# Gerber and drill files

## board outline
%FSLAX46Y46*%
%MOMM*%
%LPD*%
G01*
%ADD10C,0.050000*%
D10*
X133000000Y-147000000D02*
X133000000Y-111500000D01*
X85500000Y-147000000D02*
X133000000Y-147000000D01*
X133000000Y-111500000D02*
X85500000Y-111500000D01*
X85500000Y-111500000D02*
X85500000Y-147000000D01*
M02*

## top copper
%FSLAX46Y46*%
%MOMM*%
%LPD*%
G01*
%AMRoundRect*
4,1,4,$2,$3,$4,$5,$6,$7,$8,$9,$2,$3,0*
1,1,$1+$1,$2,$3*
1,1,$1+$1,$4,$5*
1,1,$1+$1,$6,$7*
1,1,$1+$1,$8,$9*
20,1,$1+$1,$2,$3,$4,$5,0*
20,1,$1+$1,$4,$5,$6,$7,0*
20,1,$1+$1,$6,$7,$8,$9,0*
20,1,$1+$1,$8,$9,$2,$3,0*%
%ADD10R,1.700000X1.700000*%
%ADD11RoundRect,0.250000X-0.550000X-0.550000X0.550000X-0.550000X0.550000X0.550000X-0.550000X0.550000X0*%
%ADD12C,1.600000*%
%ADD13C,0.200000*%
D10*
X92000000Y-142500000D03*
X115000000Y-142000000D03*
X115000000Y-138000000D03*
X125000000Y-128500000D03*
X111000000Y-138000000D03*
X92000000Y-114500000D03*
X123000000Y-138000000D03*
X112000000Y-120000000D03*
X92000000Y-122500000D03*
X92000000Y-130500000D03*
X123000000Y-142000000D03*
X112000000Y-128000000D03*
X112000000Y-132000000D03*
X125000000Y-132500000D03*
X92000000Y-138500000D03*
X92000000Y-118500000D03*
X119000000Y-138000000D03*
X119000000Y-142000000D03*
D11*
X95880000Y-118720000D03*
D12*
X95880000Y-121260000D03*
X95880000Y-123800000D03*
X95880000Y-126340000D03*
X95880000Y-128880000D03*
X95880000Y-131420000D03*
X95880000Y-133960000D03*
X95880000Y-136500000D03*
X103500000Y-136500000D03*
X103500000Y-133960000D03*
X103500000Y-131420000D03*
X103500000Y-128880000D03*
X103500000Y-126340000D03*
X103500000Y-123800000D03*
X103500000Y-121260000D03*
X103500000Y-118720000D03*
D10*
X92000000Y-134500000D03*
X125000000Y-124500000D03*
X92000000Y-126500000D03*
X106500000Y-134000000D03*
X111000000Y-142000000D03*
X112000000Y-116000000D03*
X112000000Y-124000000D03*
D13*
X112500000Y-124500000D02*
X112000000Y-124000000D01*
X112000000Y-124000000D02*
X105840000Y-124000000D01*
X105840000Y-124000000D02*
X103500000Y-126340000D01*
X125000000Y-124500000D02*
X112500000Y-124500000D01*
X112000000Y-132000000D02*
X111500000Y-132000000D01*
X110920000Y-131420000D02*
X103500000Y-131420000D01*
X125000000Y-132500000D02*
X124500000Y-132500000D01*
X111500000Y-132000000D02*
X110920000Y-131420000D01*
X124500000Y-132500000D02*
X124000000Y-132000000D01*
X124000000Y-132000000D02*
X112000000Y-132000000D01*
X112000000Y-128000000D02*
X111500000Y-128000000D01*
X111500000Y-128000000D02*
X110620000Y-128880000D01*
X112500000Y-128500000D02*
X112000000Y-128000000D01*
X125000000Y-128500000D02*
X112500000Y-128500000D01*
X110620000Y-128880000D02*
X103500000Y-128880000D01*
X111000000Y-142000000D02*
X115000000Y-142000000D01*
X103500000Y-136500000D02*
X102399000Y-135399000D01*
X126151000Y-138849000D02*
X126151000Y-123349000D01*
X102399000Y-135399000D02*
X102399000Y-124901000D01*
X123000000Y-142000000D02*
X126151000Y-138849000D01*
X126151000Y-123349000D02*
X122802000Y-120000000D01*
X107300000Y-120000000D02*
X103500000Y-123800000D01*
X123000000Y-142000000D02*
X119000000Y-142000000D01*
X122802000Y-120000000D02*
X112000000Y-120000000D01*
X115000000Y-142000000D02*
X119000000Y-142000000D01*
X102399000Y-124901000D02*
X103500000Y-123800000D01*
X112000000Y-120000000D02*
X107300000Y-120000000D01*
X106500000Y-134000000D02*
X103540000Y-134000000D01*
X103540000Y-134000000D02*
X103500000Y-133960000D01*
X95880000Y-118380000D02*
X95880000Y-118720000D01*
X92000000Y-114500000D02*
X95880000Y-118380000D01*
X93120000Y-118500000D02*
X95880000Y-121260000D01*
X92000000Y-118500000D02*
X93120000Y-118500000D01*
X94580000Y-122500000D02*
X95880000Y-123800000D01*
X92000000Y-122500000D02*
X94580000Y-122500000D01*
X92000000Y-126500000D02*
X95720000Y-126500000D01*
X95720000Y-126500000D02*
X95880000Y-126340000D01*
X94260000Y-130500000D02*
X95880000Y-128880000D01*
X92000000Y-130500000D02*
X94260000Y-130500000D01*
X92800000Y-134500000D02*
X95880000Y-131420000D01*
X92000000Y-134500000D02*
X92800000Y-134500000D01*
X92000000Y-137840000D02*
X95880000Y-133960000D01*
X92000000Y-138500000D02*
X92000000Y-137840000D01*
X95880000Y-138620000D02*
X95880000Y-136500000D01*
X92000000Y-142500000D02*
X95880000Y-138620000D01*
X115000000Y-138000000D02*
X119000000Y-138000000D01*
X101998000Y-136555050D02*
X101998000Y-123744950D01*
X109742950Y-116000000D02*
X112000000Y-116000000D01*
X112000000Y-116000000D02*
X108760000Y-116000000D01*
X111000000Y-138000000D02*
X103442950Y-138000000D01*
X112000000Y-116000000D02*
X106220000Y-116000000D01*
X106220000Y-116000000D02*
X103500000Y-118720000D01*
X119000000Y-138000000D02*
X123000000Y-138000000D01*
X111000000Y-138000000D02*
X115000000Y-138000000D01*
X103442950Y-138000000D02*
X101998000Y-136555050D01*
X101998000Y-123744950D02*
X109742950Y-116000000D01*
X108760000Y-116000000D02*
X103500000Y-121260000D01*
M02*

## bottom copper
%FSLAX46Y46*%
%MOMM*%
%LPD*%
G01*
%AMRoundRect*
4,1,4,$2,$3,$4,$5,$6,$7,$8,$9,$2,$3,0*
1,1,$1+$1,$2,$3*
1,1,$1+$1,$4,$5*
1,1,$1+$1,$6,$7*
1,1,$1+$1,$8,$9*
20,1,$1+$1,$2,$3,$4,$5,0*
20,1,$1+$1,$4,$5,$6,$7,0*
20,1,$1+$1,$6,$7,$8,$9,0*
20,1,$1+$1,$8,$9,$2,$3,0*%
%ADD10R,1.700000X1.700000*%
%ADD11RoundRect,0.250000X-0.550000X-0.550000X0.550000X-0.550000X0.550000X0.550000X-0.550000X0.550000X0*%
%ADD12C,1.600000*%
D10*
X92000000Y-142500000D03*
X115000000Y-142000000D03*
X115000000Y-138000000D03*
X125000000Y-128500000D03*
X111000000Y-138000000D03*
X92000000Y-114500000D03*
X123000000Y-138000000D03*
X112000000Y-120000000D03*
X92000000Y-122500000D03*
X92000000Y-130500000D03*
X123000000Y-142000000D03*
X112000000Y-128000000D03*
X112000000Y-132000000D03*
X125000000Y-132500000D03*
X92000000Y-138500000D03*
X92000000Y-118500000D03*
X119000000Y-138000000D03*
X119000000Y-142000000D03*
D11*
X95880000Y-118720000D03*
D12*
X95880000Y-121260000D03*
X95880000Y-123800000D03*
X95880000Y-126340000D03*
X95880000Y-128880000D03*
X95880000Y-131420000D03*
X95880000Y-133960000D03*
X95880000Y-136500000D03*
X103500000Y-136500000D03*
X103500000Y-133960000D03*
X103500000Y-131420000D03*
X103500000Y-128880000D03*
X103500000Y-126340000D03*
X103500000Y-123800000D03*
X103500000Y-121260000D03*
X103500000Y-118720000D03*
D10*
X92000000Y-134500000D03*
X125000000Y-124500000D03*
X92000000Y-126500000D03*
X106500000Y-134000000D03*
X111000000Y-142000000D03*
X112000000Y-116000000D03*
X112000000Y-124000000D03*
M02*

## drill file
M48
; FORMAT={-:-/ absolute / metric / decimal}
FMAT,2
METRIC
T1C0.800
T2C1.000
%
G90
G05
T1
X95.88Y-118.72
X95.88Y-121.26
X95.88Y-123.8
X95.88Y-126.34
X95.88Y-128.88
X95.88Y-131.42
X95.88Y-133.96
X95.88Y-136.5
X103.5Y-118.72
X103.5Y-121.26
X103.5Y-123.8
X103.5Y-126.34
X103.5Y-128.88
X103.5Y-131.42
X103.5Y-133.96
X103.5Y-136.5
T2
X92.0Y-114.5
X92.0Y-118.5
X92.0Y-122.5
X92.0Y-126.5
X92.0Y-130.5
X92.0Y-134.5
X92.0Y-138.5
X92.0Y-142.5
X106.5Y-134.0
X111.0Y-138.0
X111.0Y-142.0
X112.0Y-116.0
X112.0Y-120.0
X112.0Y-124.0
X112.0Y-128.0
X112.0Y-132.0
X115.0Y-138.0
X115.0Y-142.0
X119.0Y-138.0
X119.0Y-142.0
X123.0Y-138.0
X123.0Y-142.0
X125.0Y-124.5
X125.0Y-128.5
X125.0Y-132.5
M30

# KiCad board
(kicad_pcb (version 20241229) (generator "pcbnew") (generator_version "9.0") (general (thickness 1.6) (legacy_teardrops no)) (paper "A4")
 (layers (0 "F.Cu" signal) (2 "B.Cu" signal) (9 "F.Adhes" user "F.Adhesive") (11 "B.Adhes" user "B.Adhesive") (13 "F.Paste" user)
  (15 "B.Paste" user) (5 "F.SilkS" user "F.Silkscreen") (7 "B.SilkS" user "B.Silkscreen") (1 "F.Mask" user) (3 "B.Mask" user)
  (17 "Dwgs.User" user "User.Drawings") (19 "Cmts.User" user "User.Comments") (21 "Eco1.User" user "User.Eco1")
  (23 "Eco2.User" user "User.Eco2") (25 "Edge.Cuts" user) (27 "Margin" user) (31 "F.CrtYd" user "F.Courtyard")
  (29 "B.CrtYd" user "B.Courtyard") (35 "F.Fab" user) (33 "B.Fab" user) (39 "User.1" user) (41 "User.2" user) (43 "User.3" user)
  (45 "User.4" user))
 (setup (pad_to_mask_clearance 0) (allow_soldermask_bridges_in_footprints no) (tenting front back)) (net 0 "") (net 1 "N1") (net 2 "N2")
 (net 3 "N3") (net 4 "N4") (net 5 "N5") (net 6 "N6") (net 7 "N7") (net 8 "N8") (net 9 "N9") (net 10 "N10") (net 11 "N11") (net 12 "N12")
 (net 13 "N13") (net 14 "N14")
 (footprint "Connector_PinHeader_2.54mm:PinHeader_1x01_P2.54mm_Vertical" (layer "F.Cu") (at 92 142.5)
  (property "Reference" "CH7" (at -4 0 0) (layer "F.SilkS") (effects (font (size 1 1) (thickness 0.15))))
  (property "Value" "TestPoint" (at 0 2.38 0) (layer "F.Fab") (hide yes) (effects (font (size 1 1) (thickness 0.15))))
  (pad "1" thru_hole rect (at 0 0) (size 1.7 1.7) (drill 1) (layers "*.Cu" "*.Mask") (remove_unused_layers no) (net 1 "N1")))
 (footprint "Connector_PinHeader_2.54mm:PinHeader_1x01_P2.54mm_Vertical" (layer "F.Cu") (at 115 142)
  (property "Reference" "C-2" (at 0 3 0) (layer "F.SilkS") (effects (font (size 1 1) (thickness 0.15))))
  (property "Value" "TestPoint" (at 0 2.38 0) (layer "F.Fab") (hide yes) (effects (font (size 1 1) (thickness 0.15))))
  (pad "1" thru_hole rect (at 0 0) (size 1.7 1.7) (drill 1) (layers "*.Cu" "*.Mask") (remove_unused_layers no) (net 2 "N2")))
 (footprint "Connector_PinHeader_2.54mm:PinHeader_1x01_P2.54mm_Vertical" (layer "F.Cu") (at 115 138)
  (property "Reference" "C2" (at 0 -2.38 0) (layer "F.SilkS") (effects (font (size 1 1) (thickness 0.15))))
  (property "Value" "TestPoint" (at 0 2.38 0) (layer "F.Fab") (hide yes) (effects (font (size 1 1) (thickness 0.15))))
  (pad "1" thru_hole rect (at 0 0) (size 1.7 1.7) (drill 1) (layers "*.Cu" "*.Mask") (remove_unused_layers no) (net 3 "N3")))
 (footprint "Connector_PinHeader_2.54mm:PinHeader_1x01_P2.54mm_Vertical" (layer "F.Cu") (at 125 128.5)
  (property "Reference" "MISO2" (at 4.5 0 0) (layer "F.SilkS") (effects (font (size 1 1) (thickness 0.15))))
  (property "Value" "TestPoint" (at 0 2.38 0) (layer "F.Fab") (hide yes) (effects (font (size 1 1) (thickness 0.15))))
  (pad "1" thru_hole rect (at 0 0) (size 1.7 1.7) (drill 1) (layers "*.Cu" "*.Mask") (remove_unused_layers no) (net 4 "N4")))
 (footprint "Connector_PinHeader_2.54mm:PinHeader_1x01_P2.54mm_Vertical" (layer "F.Cu") (at 111 138)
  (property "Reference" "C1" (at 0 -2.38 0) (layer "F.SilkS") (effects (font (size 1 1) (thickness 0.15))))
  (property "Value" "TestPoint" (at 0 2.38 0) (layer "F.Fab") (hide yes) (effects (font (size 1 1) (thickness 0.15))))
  (pad "1" thru_hole rect (at 0 0) (size 1.7 1.7) (drill 1) (layers "*.Cu" "*.Mask") (remove_unused_layers no) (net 3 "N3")))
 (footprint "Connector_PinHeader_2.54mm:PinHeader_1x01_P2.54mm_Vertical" (layer "F.Cu") (at 92 114.5)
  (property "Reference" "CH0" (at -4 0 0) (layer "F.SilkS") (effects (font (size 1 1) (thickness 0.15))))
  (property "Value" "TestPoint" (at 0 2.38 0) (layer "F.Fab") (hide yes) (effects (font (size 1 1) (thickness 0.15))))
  (pad "1" thru_hole rect (at 0 0) (size 1.7 1.7) (drill 1) (layers "*.Cu" "*.Mask") (remove_unused_layers no) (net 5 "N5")))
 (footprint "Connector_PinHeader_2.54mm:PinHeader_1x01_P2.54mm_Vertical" (layer "F.Cu") (at 123 138)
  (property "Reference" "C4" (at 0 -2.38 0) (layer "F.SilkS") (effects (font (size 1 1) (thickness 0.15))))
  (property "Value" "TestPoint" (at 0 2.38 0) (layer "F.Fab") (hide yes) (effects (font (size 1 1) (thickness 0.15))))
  (pad "1" thru_hole rect (at 0 0) (size 1.7 1.7) (drill 1) (layers "*.Cu" "*.Mask") (remove_unused_layers no) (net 3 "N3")))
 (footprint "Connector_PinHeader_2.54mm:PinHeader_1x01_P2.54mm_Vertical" (layer "F.Cu") (at 112 120)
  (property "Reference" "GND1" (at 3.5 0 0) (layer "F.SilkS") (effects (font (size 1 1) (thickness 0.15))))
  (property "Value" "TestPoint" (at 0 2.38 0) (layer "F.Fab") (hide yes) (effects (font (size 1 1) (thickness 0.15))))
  (pad "1" thru_hole rect (at 0 0) (size 1.7 1.7) (drill 1) (layers "*.Cu" "*.Mask") (remove_unused_layers no) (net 2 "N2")))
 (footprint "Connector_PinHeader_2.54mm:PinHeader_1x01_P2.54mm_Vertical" (layer "F.Cu") (at 92 122.5)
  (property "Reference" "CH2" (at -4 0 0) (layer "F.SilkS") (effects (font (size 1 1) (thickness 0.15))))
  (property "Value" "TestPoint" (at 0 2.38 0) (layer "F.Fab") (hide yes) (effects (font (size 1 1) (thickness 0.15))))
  (pad "1" thru_hole rect (at 0 0) (size 1.7 1.7) (drill 1) (layers "*.Cu" "*.Mask") (remove_unused_layers no) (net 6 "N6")))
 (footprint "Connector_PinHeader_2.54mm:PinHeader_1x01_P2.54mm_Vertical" (layer "F.Cu") (at 92 130.5)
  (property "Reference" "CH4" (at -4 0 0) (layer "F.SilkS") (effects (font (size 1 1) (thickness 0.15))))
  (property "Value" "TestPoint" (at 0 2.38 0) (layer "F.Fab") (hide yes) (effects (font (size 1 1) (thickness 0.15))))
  (pad "1" thru_hole rect (at 0 0) (size 1.7 1.7) (drill 1) (layers "*.Cu" "*.Mask") (remove_unused_layers no) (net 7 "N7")))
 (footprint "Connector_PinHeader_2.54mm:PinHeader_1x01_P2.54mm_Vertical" (layer "F.Cu") (at 123 142)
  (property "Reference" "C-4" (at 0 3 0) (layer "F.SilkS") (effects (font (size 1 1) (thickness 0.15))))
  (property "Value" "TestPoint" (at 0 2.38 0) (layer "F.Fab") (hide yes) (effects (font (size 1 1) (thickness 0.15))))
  (pad "1" thru_hole rect (at 0 0) (size 1.7 1.7) (drill 1) (layers "*.Cu" "*.Mask") (remove_unused_layers no) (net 2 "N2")))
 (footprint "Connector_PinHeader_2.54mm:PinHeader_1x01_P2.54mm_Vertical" (layer "F.Cu") (at 112 128)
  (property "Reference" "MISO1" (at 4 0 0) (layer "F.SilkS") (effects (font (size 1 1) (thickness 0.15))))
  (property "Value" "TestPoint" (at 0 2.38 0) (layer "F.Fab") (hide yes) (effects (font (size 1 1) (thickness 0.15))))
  (pad "1" thru_hole rect (at 0 0) (size 1.7 1.7) (drill 1) (layers "*.Cu" "*.Mask") (remove_unused_layers no) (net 4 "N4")))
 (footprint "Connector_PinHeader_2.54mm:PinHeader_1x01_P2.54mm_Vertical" (layer "F.Cu") (at 112 132)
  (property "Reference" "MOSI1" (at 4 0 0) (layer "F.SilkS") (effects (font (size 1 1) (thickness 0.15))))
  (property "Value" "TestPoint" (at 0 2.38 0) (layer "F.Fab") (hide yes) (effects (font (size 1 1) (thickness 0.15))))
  (pad "1" thru_hole rect (at 0 0) (size 1.7 1.7) (drill 1) (layers "*.Cu" "*.Mask") (remove_unused_layers no) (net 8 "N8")))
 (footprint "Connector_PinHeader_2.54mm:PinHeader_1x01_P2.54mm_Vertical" (layer "F.Cu") (at 125 132.5)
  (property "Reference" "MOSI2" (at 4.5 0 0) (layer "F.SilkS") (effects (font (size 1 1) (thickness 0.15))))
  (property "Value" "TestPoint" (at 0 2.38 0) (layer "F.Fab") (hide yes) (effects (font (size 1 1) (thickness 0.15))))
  (pad "1" thru_hole rect (at 0 0) (size 1.7 1.7) (drill 1) (layers "*.Cu" "*.Mask") (remove_unused_layers no) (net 8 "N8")))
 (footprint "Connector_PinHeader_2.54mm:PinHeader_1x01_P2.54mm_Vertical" (layer "F.Cu") (at 92 138.5)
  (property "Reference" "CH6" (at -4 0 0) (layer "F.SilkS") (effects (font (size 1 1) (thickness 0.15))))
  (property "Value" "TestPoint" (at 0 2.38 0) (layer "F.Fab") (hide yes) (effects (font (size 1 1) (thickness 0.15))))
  (pad "1" thru_hole rect (at 0 0) (size 1.7 1.7) (drill 1) (layers "*.Cu" "*.Mask") (remove_unused_layers no) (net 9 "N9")))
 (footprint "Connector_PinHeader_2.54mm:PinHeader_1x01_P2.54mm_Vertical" (layer "F.Cu") (at 92 118.5)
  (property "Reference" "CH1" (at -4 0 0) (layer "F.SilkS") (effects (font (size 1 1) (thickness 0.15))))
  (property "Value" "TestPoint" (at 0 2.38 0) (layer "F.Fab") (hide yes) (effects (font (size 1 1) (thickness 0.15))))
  (pad "1" thru_hole rect (at 0 0) (size 1.7 1.7) (drill 1) (layers "*.Cu" "*.Mask") (remove_unused_layers no) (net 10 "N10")))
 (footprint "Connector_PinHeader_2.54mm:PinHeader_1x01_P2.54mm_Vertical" (layer "F.Cu") (at 119 138)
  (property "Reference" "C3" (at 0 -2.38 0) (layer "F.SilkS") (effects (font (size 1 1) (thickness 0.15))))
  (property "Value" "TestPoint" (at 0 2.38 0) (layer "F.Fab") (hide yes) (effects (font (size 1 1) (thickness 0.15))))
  (pad "1" thru_hole rect (at 0 0) (size 1.7 1.7) (drill 1) (layers "*.Cu" "*.Mask") (remove_unused_layers no) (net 3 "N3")))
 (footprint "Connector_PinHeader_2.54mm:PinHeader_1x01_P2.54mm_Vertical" (layer "F.Cu") (at 119 142)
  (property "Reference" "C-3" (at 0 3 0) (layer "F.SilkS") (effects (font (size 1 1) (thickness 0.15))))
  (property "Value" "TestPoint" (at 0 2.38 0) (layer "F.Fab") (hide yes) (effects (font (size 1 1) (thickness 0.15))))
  (pad "1" thru_hole rect (at 0 0) (size 1.7 1.7) (drill 1) (layers "*.Cu" "*.Mask") (remove_unused_layers no) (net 2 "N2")))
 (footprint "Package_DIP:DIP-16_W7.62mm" (layer "F.Cu") (at 95.88 118.72)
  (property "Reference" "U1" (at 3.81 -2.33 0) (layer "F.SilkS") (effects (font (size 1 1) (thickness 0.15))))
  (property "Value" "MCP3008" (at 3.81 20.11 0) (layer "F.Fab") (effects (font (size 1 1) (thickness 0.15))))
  (pad "1" thru_hole roundrect (at 0 0) (size 1.6 1.6) (drill 0.8) (layers "*.Cu" "*.Mask") (remove_unused_layers no)
   (roundrect_rratio 0.15625) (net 5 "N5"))
  (pad "2" thru_hole circle (at 0 2.54) (size 1.6 1.6) (drill 0.8) (layers "*.Cu" "*.Mask") (remove_unused_layers no) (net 10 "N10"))
  (pad "3" thru_hole circle (at 0 5.08) (size 1.6 1.6) (drill 0.8) (layers "*.Cu" "*.Mask") (remove_unused_layers no) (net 6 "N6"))
  (pad "4" thru_hole circle (at 0 7.62) (size 1.6 1.6) (drill 0.8) (layers "*.Cu" "*.Mask") (remove_unused_layers no) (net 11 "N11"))
  (pad "5" thru_hole circle (at 0 10.16) (size 1.6 1.6) (drill 0.8) (layers "*.Cu" "*.Mask") (remove_unused_layers no) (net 7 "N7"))
  (pad "6" thru_hole circle (at 0 12.7) (size 1.6 1.6) (drill 0.8) (layers "*.Cu" "*.Mask") (remove_unused_layers no) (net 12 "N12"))
  (pad "7" thru_hole circle (at 0 15.24) (size 1.6 1.6) (drill 0.8) (layers "*.Cu" "*.Mask") (remove_unused_layers no) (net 9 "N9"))
  (pad "8" thru_hole circle (at 0 17.78) (size 1.6 1.6) (drill 0.8) (layers "*.Cu" "*.Mask") (remove_unused_layers no) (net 1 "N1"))
  (pad "9" thru_hole circle (at 7.62 17.78) (size 1.6 1.6) (drill 0.8) (layers "*.Cu" "*.Mask") (remove_unused_layers no) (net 2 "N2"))
  (pad "10" thru_hole circle (at 7.62 15.24) (size 1.6 1.6) (drill 0.8) (layers "*.Cu" "*.Mask") (remove_unused_layers no) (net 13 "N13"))
  (pad "11" thru_hole circle (at 7.62 12.7) (size 1.6 1.6) (drill 0.8) (layers "*.Cu" "*.Mask") (remove_unused_layers no) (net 8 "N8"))
  (pad "12" thru_hole circle (at 7.62 10.16) (size 1.6 1.6) (drill 0.8) (layers "*.Cu" "*.Mask") (remove_unused_layers no) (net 4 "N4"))
  (pad "13" thru_hole circle (at 7.62 7.62) (size 1.6 1.6) (drill 0.8) (layers "*.Cu" "*.Mask") (remove_unused_layers no) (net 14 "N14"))
  (pad "14" thru_hole circle (at 7.62 5.08) (size 1.6 1.6) (drill 0.8) (layers "*.Cu" "*.Mask") (remove_unused_layers no) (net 2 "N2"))
  (pad "15" thru_hole circle (at 7.62 2.54) (size 1.6 1.6) (drill 0.8) (layers "*.Cu" "*.Mask") (remove_unused_layers no) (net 3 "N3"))
  (pad "16" thru_hole circle (at 7.62 0) (size 1.6 1.6) (drill 0.8) (layers "*.Cu" "*.Mask") (remove_unused_layers no) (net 3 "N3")))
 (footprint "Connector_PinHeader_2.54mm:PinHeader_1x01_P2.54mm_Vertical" (layer "F.Cu") (at 92 134.5)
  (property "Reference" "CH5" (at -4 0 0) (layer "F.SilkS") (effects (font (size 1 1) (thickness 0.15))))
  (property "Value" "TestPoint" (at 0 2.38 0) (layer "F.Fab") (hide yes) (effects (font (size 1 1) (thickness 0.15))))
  (pad "1" thru_hole rect (at 0 0) (size 1.7 1.7) (drill 1) (layers "*.Cu" "*.Mask") (remove_unused_layers no) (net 12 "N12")))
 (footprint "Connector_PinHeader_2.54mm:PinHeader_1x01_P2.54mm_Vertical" (layer "F.Cu") (at 125 124.5)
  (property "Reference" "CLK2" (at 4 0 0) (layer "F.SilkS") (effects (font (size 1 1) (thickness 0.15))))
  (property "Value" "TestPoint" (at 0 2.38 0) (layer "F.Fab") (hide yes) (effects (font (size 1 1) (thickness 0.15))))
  (pad "1" thru_hole rect (at 0 0) (size 1.7 1.7) (drill 1) (layers "*.Cu" "*.Mask") (remove_unused_layers no) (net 14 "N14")))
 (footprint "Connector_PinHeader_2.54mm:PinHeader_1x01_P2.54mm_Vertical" (layer "F.Cu") (at 92 126.5)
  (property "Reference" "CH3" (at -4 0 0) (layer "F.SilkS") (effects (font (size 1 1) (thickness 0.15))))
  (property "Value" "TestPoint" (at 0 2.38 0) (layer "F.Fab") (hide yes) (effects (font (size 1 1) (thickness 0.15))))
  (pad "1" thru_hole rect (at 0 0) (size 1.7 1.7) (drill 1) (layers "*.Cu" "*.Mask") (remove_unused_layers no) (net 11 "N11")))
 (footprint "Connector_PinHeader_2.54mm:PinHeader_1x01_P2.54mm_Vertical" (layer "F.Cu") (at 106.5 134)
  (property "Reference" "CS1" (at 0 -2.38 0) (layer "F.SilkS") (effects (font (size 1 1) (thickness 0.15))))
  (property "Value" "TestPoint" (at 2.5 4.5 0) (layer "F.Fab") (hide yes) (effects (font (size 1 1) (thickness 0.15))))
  (pad "1" thru_hole rect (at 0 0) (size 1.7 1.7) (drill 1) (layers "*.Cu" "*.Mask") (remove_unused_layers no) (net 13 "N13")))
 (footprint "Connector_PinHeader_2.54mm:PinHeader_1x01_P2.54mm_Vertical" (layer "F.Cu") (at 111 142)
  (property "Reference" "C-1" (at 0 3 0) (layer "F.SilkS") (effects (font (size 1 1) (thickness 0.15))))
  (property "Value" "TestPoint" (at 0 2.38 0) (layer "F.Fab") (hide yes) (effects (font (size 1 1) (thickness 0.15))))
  (pad "1" thru_hole rect (at 0 0) (size 1.7 1.7) (drill 1) (layers "*.Cu" "*.Mask") (remove_unused_layers no) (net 2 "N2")))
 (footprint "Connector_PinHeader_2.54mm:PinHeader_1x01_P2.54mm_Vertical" (layer "F.Cu") (at 112 116)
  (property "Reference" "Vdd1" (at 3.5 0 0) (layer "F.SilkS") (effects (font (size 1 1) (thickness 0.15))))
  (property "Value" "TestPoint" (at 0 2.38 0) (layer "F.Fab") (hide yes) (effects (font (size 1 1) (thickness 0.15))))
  (pad "1" thru_hole rect (at 0 0) (size 1.7 1.7) (drill 1) (layers "*.Cu" "*.Mask") (remove_unused_layers no) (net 3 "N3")))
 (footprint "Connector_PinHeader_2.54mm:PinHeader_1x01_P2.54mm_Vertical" (layer "F.Cu") (at 112 124)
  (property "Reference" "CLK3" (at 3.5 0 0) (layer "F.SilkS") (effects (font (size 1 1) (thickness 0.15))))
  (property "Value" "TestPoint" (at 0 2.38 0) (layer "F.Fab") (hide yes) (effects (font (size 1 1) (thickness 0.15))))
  (pad "1" thru_hole rect (at 0 0) (size 1.7 1.7) (drill 1) (layers "*.Cu" "*.Mask") (remove_unused_layers no) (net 14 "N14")))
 (gr_line (start 133 147) (end 133 111.5) (stroke (width 0.05) (type default)) (layer "Edge.Cuts"))
 (gr_line (start 85.5 147) (end 133 147) (stroke (width 0.05) (type default)) (layer "Edge.Cuts"))
 (gr_line (start 133 111.5) (end 85.5 111.5) (stroke (width 0.05) (type default)) (layer "Edge.Cuts"))
 (gr_line (start 85.5 111.5) (end 85.5 147) (stroke (width 0.05) (type default)) (layer "Edge.Cuts"))
 (segment (start 112.5 124.5) (end 112 124) (width 0.2) (layer "F.Cu") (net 14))
 (segment (start 112 124) (end 105.84 124) (width 0.2) (layer "F.Cu") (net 14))
 (segment (start 105.84 124) (end 103.5 126.34) (width 0.2) (layer "F.Cu") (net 14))
 (segment (start 125 124.5) (end 112.5 124.5) (width 0.2) (layer "F.Cu") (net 14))
 (segment (start 112 132) (end 111.5 132) (width 0.2) (layer "F.Cu") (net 8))
 (segment (start 110.92 131.42) (end 103.5 131.42) (width 0.2) (layer "F.Cu") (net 8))
 (segment (start 125 132.5) (end 124.5 132.5) (width 0.2) (layer "F.Cu") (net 8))
 (segment (start 111.5 132) (end 110.92 131.42) (width 0.2) (layer "F.Cu") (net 8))
 (segment (start 124.5 132.5) (end 124 132) (width 0.2) (layer "F.Cu") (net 8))
 (segment (start 124 132) (end 112 132) (width 0.2) (layer "F.Cu") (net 8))
 (segment (start 112 128) (end 111.5 128) (width 0.2) (layer "F.Cu") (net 4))
 (segment (start 111.5 128) (end 110.62 128.88) (width 0.2) (layer "F.Cu") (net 4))
 (segment (start 112.5 128.5) (end 112 128) (width 0.2) (layer "F.Cu") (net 4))
 (segment (start 125 128.5) (end 112.5 128.5) (width 0.2) (layer "F.Cu") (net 4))
 (segment (start 110.62 128.88) (end 103.5 128.88) (width 0.2) (layer "F.Cu") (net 4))
 (segment (start 111 142) (end 115 142) (width 0.2) (layer "F.Cu") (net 2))
 (segment (start 103.5 136.5) (end 102.399 135.399) (width 0.2) (layer "F.Cu") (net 2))
 (segment (start 126.151 138.849) (end 126.151 123.349) (width 0.2) (layer "F.Cu") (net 2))
 (segment (start 102.399 135.399) (end 102.399 124.901) (width 0.2) (layer "F.Cu") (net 2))
 (segment (start 123 142) (end 126.151 138.849) (width 0.2) (layer "F.Cu") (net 2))
 (segment (start 126.151 123.349) (end 122.802 120) (width 0.2) (layer "F.Cu") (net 2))
 (segment (start 107.3 120) (end 103.5 123.8) (width 0.2) (layer "F.Cu") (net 2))
 (segment (start 123 142) (end 119 142) (width 0.2) (layer "F.Cu") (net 2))
 (segment (start 122.802 120) (end 112 120) (width 0.2) (layer "F.Cu") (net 2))
 (segment (start 115 142) (end 119 142) (width 0.2) (layer "F.Cu") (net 2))
 (segment (start 102.399 124.901) (end 103.5 123.8) (width 0.2) (layer "F.Cu") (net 2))
 (segment (start 112 120) (end 107.3 120) (width 0.2) (layer "F.Cu") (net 2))
 (segment (start 106.5 134) (end 103.54 134) (width 0.2) (layer "F.Cu") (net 13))
 (segment (start 103.54 134) (end 103.5 133.96) (width 0.2) (layer "F.Cu") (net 13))
 (segment (start 95.88 118.38) (end 95.88 118.72) (width 0.2) (layer "F.Cu") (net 5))
 (segment (start 92 114.5) (end 95.88 118.38) (width 0.2) (layer "F.Cu") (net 5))
 (segment (start 93.12 118.5) (end 95.88 121.26) (width 0.2) (layer "F.Cu") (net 10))
 (segment (start 92 118.5) (end 93.12 118.5) (width 0.2) (layer "F.Cu") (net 10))
 (segment (start 94.58 122.5) (end 95.88 123.8) (width 0.2) (layer "F.Cu") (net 6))
 (segment (start 92 122.5) (end 94.58 122.5) (width 0.2) (layer "F.Cu") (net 6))
 (segment (start 92 126.5) (end 95.72 126.5) (width 0.2) (layer "F.Cu") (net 11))
 (segment (start 95.72 126.5) (end 95.88 126.34) (width 0.2) (layer "F.Cu") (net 11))
 (segment (start 94.26 130.5) (end 95.88 128.88) (width 0.2) (layer "F.Cu") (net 7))
 (segment (start 92 130.5) (end 94.26 130.5) (width 0.2) (layer "F.Cu") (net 7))
 (segment (start 92.8 134.5) (end 95.88 131.42) (width 0.2) (layer "F.Cu") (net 12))
 (segment (start 92 134.5) (end 92.8 134.5) (width 0.2) (layer "F.Cu") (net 12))
 (segment (start 92 137.84) (end 95.88 133.96) (width 0.2) (layer "F.Cu") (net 9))
 (segment (start 92 138.5) (end 92 137.84) (width 0.2) (layer "F.Cu") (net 9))
 (segment (start 95.88 138.62) (end 95.88 136.5) (width 0.2) (layer "F.Cu") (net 1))
 (segment (start 92 142.5) (end 95.88 138.62) (width 0.2) (layer "F.Cu") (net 1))
 (segment (start 115 138) (end 119 138) (width 0.2) (layer "F.Cu") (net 3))
 (segment (start 101.998 136.55505) (end 101.998 123.74495) (width 0.2) (layer "F.Cu") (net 3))
 (segment (start 109.74295 116) (end 112 116) (width 0.2) (layer "F.Cu") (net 3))
 (segment (start 112 116) (end 108.76 116) (width 0.2) (layer "F.Cu") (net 3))
 (segment (start 111 138) (end 103.44295 138) (width 0.2) (layer "F.Cu") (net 3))
 (segment (start 112 116) (end 106.22 116) (width 0.2) (layer "F.Cu") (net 3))
 (segment (start 106.22 116) (end 103.5 118.72) (width 0.2) (layer "F.Cu") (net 3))
 (segment (start 119 138) (end 123 138) (width 0.2) (layer "F.Cu") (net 3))
 (segment (start 111 138) (end 115 138) (width 0.2) (layer "F.Cu") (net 3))
 (segment (start 103.44295 138) (end 101.998 136.55505) (width 0.2) (layer "F.Cu") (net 3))
 (segment (start 101.998 123.74495) (end 109.74295 116) (width 0.2) (layer "F.Cu") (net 3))
 (segment (start 108.76 116) (end 103.5 121.26) (width 0.2) (layer "F.Cu") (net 3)))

